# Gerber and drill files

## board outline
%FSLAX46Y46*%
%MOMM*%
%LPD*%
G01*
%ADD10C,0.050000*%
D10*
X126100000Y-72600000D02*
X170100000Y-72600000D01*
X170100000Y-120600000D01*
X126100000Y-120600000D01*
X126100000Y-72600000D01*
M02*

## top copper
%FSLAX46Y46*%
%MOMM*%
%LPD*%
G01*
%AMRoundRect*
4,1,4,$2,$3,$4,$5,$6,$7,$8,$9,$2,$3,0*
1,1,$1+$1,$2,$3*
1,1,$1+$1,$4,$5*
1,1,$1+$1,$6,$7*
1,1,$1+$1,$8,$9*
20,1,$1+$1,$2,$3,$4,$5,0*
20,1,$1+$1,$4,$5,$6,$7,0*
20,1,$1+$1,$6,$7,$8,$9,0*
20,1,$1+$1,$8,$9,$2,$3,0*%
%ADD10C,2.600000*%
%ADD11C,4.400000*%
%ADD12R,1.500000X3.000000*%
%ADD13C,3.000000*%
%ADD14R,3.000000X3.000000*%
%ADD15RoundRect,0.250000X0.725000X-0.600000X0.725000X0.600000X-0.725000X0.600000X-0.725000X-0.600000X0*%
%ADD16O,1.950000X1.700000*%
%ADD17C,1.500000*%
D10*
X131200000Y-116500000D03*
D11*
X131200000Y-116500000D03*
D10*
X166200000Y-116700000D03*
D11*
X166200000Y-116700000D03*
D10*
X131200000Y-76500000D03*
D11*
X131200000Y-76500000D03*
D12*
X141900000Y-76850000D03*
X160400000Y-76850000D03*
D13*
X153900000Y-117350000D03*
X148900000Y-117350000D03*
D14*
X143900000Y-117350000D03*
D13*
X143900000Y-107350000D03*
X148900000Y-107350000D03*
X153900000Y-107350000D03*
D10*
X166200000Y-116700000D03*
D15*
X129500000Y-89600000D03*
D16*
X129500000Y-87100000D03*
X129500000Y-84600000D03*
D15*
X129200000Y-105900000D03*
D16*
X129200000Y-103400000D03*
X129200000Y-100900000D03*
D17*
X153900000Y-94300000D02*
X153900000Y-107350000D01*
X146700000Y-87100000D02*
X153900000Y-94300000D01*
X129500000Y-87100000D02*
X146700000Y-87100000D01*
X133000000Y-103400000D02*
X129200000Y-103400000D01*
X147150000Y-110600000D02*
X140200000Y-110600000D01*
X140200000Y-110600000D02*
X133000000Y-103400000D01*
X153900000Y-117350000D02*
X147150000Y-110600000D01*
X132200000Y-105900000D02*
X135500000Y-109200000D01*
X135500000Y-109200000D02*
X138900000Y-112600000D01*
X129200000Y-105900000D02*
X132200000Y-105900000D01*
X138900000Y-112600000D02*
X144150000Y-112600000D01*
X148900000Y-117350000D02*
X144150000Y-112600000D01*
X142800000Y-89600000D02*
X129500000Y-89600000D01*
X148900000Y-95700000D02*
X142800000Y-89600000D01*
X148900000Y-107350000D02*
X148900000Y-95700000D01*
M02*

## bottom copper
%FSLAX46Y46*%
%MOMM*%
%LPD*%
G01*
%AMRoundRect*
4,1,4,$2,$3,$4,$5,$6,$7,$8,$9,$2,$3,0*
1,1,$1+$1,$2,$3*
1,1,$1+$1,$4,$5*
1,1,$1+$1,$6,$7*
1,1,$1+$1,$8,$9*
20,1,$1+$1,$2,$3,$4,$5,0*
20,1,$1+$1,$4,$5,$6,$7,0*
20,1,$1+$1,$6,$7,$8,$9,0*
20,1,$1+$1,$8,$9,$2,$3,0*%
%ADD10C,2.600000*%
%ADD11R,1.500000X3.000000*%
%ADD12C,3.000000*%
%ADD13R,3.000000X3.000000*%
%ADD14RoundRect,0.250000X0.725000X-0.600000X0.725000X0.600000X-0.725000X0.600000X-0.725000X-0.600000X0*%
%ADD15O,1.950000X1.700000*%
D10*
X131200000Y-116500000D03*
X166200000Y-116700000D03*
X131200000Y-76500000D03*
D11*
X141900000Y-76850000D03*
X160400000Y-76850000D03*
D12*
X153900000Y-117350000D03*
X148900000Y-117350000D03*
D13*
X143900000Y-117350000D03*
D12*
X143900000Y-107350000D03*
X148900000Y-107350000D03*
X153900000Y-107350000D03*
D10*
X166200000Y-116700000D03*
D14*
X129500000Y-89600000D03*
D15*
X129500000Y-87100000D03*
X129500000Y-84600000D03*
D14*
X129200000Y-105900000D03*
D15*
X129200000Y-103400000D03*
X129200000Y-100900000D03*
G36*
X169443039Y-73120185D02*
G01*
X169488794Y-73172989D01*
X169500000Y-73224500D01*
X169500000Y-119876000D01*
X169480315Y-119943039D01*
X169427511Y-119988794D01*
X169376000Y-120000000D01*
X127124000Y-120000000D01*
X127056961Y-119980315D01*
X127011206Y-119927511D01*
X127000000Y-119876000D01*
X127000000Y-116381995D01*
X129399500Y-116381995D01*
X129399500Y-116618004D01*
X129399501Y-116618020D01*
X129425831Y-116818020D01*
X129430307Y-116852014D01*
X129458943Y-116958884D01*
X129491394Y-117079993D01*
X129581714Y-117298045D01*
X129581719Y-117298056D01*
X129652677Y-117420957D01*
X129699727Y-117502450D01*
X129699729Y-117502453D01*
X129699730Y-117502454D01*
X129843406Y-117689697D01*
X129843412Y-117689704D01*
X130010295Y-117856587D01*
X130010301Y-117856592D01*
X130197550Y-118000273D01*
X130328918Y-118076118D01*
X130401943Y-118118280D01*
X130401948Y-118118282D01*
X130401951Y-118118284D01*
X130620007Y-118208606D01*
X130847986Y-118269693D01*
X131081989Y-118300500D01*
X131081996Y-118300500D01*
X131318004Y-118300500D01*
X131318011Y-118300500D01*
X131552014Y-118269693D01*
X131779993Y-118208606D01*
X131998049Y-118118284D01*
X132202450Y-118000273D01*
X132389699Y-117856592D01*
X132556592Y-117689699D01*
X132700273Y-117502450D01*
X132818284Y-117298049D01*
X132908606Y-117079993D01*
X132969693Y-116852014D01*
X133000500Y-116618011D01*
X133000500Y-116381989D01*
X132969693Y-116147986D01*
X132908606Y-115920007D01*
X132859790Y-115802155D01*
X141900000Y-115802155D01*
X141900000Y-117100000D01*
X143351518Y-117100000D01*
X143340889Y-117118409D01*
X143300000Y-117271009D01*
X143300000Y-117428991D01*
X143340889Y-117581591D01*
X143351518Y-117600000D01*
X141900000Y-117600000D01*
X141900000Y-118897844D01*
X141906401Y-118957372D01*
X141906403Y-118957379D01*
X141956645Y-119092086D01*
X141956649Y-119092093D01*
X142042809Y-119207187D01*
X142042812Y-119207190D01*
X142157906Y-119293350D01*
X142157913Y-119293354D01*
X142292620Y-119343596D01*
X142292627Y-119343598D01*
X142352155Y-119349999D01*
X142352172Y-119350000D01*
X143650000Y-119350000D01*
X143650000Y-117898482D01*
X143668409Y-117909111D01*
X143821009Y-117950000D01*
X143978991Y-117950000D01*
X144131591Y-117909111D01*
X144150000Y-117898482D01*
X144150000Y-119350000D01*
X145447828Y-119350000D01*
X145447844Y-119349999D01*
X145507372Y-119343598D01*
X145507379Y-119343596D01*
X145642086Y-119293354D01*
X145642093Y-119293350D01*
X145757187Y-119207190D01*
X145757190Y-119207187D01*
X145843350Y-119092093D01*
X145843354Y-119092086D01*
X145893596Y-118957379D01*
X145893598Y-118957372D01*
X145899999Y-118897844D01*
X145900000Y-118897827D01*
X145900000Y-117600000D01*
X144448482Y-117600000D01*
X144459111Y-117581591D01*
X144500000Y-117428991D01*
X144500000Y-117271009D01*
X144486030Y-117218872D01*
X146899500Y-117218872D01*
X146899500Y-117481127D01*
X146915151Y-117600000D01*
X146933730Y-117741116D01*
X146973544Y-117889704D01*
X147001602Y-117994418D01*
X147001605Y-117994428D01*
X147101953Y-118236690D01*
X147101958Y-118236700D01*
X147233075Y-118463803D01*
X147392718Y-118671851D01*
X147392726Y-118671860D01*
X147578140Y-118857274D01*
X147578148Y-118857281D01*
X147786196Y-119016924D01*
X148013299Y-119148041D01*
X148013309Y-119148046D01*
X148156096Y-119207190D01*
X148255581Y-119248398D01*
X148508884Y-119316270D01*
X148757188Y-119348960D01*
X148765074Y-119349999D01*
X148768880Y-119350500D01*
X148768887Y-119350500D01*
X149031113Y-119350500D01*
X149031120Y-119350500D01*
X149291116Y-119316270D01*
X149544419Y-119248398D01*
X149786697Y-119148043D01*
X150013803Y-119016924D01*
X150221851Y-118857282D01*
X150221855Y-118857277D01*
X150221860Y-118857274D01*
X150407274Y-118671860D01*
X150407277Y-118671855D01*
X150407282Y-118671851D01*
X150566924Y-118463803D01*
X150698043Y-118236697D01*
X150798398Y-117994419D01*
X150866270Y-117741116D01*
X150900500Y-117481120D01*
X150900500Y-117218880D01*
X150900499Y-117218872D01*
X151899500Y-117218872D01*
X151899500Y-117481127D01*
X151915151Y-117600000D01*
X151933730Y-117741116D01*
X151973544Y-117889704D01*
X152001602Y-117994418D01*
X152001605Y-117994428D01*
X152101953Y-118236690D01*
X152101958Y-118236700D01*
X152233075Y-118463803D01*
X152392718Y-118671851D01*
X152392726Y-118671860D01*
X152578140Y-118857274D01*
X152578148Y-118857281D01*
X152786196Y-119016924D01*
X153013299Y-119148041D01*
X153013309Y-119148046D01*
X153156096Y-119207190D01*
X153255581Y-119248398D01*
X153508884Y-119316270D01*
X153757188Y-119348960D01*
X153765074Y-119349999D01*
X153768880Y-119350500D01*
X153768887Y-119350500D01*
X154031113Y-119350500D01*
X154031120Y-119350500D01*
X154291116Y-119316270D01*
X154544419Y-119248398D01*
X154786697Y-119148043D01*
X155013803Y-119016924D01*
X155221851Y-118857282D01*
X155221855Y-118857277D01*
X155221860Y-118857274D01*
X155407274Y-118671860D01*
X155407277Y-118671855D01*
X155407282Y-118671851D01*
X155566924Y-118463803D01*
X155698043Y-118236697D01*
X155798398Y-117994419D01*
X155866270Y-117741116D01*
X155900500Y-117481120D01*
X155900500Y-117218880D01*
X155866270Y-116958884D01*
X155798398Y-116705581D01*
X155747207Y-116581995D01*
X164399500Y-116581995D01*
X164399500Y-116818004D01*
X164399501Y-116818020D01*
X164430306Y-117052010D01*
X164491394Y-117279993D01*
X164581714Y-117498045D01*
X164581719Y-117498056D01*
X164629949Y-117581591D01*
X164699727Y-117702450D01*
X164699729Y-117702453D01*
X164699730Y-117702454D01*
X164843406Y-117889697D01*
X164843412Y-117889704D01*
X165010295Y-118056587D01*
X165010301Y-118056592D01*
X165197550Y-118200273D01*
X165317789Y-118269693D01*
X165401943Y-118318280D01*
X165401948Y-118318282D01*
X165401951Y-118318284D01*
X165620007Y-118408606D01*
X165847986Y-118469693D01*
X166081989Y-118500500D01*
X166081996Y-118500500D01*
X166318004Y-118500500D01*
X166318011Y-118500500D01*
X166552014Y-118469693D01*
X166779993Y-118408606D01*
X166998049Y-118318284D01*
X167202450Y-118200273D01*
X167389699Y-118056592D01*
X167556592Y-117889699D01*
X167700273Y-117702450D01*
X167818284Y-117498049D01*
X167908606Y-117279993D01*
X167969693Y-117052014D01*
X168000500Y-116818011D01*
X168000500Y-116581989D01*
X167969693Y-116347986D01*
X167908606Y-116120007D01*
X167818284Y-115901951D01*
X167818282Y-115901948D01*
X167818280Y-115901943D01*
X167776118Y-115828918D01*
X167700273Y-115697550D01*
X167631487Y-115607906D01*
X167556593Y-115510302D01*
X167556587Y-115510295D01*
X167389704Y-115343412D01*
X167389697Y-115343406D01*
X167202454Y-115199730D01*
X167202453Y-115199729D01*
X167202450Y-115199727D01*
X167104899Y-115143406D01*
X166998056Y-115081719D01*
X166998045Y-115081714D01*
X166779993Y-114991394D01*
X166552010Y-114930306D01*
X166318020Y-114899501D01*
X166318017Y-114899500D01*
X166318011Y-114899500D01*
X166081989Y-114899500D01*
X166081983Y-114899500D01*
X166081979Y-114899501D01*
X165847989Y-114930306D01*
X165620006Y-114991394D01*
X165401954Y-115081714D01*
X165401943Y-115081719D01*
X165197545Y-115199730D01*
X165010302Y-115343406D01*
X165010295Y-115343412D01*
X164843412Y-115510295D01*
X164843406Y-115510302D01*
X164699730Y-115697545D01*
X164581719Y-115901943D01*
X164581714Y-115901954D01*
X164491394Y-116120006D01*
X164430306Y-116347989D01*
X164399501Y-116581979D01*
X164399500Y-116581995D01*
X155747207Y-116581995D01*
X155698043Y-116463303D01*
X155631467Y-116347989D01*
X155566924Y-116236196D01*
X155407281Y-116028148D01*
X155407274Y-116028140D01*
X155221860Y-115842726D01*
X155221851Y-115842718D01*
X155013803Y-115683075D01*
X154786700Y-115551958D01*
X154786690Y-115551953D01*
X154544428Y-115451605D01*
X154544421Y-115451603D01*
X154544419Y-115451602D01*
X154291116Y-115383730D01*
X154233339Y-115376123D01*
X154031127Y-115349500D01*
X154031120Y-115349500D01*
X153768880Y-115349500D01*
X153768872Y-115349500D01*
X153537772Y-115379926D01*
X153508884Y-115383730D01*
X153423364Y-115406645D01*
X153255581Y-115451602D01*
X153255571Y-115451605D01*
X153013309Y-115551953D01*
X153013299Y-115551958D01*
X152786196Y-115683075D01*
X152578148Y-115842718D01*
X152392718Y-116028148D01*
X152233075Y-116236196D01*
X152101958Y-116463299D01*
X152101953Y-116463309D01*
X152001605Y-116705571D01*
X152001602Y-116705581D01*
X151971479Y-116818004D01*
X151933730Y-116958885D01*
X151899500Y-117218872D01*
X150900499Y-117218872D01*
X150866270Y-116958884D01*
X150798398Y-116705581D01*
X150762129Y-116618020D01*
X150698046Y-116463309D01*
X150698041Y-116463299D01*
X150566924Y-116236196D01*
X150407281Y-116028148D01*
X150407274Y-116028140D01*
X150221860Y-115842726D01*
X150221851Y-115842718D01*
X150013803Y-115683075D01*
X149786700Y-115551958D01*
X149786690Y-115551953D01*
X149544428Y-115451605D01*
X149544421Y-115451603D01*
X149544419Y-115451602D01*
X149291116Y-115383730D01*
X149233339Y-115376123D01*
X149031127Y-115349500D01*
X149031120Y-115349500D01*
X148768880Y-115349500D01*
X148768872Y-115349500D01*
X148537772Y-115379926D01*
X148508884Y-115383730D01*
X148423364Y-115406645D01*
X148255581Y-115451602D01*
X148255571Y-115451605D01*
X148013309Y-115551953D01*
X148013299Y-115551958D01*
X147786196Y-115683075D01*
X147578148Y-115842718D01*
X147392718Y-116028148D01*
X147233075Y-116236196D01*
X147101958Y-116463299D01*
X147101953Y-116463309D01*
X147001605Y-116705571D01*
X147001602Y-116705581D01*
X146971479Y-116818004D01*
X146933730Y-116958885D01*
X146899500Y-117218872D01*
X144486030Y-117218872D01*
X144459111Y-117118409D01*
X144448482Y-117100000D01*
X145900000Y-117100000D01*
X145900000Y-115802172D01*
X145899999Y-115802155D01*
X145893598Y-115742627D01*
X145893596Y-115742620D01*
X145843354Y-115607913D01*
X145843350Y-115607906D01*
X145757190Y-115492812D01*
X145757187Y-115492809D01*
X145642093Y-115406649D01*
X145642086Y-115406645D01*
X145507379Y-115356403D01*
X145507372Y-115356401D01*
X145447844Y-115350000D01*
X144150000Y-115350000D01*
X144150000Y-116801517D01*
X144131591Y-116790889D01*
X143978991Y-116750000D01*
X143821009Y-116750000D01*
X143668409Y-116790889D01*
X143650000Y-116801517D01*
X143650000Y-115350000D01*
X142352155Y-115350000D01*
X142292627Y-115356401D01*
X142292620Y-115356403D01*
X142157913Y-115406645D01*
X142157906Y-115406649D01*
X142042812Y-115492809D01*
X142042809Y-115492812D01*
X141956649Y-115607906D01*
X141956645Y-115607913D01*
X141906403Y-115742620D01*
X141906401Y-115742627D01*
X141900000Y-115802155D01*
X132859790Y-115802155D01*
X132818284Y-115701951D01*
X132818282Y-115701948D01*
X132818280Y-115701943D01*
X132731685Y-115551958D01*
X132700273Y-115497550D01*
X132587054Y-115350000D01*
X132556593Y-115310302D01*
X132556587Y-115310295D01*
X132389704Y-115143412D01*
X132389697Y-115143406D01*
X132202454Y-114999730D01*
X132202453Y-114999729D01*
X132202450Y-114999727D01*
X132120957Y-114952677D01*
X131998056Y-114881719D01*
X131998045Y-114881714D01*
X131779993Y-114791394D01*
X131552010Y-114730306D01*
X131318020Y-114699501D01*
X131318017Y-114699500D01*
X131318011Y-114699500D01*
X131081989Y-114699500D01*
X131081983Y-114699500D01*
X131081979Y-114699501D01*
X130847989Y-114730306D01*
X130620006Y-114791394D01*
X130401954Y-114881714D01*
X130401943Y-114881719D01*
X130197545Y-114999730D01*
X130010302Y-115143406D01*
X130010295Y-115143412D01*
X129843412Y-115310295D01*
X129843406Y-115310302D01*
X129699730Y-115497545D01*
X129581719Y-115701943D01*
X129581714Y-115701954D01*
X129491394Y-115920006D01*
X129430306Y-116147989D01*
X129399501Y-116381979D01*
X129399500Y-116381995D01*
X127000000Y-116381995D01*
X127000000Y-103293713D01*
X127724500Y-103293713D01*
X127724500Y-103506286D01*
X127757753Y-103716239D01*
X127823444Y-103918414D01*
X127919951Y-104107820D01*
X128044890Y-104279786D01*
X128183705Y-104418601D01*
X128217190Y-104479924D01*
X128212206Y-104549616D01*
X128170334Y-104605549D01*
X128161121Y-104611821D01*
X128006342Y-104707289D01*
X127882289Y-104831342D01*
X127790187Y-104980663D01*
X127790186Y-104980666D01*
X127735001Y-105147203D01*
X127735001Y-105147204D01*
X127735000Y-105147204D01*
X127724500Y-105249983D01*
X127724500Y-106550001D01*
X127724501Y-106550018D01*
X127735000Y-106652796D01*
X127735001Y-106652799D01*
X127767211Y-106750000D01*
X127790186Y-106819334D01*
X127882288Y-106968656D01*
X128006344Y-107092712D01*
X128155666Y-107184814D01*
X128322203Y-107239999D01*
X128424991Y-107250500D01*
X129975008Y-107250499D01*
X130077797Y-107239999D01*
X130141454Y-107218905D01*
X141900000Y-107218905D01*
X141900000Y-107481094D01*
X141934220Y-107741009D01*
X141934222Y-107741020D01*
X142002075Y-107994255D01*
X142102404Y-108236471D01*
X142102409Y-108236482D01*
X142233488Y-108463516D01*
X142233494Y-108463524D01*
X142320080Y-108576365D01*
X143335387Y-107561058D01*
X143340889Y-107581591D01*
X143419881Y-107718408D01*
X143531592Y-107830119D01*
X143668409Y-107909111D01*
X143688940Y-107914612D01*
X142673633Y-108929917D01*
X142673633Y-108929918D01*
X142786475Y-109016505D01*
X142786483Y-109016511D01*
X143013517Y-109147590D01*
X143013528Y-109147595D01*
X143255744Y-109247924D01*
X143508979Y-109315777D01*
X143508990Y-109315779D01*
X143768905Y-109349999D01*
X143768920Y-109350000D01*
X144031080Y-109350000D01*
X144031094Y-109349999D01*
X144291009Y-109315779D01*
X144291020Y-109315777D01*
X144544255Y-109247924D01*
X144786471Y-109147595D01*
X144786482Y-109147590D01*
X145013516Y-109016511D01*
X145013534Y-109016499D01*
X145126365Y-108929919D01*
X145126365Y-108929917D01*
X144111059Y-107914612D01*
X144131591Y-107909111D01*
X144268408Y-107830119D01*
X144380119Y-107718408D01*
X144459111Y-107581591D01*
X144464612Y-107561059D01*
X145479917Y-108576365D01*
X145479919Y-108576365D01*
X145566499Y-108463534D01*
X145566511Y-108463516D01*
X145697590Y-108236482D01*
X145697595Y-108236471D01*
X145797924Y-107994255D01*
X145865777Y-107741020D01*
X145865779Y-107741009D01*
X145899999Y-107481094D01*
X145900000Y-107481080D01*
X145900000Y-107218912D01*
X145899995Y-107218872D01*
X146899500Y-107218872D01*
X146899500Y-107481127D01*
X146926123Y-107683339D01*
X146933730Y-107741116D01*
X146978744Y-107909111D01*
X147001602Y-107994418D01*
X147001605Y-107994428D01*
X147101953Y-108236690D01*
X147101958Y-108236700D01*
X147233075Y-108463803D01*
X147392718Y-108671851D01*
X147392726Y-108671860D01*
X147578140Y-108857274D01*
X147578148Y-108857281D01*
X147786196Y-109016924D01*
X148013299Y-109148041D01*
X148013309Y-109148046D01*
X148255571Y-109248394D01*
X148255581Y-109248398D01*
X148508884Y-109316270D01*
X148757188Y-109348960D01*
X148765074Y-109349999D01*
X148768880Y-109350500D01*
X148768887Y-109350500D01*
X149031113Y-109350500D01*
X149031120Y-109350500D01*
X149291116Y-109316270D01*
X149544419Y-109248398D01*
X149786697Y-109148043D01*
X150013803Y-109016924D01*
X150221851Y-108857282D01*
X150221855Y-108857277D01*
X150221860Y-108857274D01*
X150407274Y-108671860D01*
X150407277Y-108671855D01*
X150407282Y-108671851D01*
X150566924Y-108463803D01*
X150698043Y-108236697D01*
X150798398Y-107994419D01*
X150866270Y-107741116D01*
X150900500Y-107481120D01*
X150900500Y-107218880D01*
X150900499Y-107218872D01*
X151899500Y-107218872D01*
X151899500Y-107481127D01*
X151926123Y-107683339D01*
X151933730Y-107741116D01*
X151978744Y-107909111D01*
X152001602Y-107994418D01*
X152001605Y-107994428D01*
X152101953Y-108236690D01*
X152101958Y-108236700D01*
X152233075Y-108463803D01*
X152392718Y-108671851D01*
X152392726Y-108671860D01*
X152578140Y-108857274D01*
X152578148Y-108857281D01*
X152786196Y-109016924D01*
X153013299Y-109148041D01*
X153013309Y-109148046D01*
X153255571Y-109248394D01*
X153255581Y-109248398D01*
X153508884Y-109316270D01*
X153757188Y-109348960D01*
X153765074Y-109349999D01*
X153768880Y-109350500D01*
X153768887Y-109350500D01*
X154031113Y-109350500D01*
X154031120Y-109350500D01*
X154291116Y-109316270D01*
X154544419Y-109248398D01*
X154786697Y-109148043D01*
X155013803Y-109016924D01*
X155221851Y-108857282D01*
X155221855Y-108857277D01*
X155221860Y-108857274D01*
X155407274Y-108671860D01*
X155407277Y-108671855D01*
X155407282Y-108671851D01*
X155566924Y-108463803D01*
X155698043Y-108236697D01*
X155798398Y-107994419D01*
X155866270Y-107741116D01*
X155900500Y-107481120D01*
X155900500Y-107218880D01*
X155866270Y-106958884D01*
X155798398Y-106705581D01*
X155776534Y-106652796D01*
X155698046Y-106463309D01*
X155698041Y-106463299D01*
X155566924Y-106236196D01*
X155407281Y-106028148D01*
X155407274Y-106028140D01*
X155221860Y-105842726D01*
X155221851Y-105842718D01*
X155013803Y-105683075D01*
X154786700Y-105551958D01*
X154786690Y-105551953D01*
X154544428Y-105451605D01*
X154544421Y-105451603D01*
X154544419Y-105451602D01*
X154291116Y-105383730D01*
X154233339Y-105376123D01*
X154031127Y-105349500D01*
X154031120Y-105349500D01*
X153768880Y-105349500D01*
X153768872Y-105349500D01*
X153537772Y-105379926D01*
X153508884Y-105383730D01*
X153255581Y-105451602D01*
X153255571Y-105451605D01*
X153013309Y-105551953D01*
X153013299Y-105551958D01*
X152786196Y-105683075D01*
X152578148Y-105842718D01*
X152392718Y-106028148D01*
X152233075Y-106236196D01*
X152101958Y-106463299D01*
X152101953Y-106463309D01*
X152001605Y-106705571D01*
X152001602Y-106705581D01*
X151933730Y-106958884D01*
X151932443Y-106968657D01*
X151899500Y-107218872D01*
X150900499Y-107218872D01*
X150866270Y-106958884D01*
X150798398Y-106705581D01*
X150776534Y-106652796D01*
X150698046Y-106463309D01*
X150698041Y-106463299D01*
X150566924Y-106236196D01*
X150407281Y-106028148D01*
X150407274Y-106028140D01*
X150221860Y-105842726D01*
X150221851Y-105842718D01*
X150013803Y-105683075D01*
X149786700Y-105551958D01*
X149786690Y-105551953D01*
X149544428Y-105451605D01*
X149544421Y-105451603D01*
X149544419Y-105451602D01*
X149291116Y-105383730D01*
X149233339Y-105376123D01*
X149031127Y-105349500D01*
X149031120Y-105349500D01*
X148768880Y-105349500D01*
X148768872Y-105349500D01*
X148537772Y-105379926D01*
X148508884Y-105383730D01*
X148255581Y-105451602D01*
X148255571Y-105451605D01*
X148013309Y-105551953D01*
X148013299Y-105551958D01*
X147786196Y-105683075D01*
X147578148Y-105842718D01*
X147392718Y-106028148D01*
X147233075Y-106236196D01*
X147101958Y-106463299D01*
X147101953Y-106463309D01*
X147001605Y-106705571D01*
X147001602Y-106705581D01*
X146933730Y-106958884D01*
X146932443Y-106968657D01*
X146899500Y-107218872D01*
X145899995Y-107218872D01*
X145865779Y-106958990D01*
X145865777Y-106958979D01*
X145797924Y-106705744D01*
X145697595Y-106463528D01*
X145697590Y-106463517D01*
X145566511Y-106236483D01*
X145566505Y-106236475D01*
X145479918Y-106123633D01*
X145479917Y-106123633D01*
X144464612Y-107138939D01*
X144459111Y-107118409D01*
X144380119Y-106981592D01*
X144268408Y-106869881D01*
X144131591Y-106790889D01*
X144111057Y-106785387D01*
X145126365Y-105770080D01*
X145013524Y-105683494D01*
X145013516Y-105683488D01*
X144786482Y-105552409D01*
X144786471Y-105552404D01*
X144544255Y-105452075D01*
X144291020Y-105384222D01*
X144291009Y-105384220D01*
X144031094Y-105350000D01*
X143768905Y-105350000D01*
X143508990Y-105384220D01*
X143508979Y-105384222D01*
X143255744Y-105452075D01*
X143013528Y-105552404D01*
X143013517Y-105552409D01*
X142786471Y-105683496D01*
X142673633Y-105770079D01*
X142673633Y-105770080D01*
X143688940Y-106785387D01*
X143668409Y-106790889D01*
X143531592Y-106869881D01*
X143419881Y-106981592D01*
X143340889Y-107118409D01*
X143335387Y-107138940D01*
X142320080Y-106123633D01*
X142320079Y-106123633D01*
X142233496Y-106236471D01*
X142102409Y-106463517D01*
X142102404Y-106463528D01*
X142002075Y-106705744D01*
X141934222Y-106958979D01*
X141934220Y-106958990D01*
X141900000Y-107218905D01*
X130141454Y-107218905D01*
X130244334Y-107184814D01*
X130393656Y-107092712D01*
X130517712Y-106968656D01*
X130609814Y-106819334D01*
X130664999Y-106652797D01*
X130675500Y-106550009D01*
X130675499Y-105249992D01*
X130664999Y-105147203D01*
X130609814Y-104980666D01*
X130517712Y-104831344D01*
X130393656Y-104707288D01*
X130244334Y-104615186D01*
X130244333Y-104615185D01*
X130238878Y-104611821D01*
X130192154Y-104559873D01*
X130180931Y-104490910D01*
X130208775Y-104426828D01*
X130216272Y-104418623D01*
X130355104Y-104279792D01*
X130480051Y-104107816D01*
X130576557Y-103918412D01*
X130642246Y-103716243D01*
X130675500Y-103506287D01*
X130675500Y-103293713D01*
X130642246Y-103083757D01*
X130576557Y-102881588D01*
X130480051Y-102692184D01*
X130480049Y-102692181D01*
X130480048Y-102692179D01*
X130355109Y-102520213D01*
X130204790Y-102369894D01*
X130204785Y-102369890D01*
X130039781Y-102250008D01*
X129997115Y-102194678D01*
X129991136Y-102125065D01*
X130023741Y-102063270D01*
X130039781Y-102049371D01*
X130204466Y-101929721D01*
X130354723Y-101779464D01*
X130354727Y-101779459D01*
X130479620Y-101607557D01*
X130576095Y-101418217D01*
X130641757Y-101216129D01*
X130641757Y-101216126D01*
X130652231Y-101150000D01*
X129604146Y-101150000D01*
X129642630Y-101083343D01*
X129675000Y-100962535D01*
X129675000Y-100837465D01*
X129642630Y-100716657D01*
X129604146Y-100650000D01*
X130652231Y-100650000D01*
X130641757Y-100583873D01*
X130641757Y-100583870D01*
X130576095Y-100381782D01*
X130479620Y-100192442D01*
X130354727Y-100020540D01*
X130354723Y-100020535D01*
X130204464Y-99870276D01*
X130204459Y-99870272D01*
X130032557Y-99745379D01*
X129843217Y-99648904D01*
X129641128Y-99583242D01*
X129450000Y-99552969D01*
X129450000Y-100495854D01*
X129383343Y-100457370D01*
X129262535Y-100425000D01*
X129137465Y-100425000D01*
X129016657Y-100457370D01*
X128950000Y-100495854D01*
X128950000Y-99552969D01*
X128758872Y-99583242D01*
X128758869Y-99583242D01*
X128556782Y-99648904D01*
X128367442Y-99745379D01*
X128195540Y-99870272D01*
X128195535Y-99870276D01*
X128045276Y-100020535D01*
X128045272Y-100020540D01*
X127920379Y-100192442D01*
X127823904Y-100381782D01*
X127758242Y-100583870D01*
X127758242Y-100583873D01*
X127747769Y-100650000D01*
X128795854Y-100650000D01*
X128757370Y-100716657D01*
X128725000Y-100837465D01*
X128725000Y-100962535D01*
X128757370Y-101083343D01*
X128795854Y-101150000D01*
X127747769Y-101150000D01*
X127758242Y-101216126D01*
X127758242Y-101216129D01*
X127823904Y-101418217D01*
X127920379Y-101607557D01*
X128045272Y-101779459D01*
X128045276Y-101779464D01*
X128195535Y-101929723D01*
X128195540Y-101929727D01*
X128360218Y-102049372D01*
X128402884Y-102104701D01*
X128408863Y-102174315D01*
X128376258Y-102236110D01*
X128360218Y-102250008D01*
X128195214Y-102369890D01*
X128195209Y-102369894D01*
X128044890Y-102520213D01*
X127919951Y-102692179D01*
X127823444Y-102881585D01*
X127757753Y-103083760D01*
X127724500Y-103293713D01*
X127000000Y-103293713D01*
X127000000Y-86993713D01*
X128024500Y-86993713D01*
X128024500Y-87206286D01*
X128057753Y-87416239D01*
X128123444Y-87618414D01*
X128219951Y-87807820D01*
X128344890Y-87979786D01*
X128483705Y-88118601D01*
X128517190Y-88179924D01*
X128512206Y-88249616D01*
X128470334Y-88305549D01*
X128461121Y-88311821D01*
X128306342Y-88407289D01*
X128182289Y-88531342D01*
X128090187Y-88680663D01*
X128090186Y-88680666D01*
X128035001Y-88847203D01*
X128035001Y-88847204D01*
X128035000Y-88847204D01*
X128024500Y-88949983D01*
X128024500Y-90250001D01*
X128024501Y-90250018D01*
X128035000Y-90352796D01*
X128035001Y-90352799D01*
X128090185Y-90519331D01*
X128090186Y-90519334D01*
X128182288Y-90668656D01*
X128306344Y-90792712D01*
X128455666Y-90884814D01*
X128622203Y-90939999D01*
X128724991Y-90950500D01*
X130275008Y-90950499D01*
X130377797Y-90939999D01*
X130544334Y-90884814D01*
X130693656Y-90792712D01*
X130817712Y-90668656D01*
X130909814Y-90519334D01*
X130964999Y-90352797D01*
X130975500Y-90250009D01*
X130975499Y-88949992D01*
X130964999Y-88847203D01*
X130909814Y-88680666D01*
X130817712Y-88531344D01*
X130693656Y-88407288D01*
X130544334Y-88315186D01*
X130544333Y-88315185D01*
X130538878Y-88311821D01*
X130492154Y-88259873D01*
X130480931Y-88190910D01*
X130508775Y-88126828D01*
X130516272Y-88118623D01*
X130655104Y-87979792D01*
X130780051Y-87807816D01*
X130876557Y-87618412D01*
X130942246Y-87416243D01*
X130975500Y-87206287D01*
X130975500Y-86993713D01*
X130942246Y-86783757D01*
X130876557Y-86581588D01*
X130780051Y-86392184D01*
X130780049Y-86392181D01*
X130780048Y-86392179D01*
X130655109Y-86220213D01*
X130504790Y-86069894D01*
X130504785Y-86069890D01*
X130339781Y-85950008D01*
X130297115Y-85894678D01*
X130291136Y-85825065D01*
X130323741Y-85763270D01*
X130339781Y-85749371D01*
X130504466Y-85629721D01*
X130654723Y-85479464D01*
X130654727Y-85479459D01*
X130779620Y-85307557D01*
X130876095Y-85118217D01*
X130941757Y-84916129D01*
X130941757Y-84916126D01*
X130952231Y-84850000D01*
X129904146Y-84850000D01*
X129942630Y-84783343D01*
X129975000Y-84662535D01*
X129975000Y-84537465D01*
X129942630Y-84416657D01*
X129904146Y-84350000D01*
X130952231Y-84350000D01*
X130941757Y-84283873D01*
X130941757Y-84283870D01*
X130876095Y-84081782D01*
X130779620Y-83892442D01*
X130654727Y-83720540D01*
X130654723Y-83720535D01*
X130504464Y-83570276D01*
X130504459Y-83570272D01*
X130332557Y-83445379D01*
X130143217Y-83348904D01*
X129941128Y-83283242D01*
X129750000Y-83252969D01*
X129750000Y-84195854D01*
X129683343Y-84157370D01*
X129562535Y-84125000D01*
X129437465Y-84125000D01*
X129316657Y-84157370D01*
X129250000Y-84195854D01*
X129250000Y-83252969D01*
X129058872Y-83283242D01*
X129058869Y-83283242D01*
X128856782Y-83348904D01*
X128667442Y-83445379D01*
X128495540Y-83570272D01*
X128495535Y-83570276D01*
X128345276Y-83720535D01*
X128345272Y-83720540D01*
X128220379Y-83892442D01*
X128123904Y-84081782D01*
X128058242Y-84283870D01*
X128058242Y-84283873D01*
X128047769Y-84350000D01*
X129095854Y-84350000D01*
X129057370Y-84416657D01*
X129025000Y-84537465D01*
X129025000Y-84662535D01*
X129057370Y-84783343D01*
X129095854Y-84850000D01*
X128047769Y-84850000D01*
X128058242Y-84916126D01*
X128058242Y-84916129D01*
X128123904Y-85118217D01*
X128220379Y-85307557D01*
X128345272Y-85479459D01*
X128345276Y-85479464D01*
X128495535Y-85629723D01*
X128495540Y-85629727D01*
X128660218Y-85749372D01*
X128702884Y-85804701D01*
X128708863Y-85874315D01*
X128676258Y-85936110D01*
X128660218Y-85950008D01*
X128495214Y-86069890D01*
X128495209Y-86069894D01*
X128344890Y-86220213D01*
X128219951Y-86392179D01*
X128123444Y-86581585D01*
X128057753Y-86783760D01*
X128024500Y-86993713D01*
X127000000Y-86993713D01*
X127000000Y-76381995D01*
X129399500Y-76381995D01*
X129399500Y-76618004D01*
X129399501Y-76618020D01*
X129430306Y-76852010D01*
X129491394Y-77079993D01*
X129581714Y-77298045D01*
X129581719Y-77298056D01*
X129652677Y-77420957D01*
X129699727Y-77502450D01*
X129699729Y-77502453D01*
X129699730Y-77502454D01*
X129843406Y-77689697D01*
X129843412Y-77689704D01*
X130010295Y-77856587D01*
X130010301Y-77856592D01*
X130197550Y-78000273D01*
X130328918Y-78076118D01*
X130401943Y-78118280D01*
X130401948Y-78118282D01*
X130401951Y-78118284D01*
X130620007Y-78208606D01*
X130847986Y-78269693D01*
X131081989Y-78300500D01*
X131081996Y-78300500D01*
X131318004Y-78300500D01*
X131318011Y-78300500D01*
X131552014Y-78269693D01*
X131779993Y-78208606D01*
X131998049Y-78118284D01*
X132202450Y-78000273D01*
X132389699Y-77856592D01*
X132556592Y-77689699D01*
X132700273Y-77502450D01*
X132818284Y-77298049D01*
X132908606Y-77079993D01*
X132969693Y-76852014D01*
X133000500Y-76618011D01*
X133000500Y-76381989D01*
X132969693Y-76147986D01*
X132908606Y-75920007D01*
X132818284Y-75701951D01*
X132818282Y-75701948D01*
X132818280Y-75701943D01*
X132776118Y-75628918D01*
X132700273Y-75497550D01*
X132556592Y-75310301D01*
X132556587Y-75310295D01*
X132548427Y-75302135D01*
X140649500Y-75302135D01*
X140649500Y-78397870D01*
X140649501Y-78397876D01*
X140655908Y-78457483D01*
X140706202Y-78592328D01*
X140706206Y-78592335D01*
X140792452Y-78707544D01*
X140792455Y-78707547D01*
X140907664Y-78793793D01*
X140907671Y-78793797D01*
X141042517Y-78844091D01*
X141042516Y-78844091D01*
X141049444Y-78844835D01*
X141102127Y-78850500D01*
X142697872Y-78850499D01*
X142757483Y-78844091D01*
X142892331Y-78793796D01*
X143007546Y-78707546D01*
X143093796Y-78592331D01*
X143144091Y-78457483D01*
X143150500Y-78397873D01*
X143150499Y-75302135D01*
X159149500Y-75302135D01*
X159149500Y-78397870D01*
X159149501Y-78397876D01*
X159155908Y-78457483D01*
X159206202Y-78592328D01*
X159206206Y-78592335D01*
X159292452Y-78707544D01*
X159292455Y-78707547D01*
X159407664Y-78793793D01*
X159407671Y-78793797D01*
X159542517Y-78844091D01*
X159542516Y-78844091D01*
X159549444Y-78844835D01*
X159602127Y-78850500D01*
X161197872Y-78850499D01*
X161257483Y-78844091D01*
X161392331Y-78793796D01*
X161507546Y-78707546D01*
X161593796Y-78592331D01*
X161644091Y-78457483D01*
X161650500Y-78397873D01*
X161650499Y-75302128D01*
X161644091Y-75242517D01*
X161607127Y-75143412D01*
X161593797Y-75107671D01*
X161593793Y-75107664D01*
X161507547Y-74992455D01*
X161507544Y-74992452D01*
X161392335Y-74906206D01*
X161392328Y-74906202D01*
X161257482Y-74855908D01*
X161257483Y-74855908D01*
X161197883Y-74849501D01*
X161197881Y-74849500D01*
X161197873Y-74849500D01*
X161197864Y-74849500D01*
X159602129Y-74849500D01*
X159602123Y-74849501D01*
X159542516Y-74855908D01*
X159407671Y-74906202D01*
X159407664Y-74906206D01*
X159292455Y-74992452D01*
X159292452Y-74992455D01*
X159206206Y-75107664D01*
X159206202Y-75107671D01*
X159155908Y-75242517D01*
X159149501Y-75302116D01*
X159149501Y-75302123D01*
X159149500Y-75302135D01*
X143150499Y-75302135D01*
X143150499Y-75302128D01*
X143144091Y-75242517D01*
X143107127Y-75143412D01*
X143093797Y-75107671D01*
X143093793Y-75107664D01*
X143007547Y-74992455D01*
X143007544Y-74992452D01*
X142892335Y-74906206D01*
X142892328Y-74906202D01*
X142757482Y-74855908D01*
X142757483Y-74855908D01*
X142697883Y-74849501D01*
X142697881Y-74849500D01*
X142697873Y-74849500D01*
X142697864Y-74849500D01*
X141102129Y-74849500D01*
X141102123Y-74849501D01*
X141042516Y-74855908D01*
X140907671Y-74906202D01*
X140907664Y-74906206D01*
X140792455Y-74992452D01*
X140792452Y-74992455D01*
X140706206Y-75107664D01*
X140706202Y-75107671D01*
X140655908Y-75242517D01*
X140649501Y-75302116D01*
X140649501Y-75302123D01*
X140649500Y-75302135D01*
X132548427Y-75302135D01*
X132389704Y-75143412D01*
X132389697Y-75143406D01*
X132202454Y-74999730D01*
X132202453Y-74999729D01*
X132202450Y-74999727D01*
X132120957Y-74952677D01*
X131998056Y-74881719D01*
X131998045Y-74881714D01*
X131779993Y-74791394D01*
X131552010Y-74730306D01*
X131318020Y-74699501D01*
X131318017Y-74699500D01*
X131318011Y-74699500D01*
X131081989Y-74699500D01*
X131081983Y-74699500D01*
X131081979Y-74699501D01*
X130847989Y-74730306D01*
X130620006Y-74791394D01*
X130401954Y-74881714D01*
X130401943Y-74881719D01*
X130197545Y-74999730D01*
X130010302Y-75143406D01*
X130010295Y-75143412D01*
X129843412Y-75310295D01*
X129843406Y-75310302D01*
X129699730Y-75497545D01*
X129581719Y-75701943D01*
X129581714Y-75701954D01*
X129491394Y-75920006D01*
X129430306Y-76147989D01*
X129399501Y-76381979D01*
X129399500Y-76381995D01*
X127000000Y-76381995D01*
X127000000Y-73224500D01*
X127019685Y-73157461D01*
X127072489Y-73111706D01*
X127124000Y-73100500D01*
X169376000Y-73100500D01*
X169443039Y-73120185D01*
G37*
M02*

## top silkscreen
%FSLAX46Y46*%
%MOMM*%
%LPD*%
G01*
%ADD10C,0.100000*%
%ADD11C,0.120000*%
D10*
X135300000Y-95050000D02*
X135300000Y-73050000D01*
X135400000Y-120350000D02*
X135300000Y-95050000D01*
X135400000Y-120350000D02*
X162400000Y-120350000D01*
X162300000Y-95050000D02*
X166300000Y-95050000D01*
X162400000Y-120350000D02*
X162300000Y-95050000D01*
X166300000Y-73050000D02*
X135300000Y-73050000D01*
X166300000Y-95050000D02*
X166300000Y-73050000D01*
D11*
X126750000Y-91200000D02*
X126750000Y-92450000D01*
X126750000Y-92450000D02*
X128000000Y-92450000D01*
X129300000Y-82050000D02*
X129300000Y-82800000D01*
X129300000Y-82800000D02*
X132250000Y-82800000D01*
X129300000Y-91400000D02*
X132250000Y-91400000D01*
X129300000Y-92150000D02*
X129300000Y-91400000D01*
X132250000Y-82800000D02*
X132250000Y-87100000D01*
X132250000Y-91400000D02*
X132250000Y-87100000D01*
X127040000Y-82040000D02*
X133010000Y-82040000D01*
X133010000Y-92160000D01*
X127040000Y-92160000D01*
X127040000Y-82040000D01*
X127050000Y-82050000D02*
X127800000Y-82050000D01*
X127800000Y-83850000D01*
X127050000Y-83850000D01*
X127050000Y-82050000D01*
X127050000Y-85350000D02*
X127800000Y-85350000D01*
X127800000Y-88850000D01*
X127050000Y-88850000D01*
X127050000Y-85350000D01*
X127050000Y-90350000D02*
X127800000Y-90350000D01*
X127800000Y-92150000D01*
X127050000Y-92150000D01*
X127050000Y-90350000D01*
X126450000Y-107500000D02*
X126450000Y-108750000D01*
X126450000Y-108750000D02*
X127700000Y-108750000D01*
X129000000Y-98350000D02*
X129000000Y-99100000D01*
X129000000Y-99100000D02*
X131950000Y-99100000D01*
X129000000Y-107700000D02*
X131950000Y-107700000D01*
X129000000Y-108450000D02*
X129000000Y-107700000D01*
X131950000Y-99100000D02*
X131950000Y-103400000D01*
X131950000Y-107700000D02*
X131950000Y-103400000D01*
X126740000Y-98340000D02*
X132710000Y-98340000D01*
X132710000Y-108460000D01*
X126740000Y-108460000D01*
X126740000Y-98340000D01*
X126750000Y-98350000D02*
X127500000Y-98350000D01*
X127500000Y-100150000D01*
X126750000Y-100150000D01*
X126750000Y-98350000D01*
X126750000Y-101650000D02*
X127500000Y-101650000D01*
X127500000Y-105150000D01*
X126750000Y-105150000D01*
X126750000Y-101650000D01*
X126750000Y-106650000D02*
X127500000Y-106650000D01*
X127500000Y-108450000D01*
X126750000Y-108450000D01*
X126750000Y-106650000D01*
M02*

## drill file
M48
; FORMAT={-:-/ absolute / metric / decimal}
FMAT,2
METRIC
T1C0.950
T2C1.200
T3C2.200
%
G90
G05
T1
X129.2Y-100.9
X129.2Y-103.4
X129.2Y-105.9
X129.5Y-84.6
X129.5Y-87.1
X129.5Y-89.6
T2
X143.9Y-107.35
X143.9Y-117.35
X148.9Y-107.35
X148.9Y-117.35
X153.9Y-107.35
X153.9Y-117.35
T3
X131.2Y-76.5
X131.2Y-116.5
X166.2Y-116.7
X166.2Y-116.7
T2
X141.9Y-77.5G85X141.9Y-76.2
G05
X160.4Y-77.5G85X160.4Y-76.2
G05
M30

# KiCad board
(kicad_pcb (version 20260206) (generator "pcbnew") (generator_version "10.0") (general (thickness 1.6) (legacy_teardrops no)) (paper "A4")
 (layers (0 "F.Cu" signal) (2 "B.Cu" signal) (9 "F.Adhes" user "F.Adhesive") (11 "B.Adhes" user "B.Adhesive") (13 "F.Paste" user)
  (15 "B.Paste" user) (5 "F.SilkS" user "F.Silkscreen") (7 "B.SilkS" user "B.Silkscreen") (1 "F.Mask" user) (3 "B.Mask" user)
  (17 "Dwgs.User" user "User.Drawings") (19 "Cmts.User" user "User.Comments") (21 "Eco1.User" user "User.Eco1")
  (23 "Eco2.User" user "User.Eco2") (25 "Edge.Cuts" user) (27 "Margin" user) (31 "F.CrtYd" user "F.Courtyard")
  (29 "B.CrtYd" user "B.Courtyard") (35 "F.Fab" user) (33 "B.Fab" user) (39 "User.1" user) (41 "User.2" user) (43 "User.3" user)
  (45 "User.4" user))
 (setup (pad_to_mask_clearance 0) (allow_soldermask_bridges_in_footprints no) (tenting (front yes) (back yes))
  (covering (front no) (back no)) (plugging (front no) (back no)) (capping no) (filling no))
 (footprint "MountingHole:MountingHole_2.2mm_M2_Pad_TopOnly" (layer "F.Cu") (at 131.2 116.5)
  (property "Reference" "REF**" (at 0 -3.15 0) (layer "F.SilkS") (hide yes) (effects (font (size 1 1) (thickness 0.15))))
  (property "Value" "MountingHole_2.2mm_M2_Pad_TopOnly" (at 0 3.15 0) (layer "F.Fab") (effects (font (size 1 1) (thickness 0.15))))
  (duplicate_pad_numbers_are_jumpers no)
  (pad "1" thru_hole circle (at 0 0) (size 2.6 2.6) (drill 2.2) (layers "*.Cu" "*.Mask") (remove_unused_layers no) (zone_connect 2))
  (pad "1" connect circle (at 0 0) (size 4.4 4.4) (layers "F.Cu" "F.Mask") (zone_connect 2)))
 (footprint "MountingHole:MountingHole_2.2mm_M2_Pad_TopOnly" (layer "F.Cu") (at 166.2 116.7)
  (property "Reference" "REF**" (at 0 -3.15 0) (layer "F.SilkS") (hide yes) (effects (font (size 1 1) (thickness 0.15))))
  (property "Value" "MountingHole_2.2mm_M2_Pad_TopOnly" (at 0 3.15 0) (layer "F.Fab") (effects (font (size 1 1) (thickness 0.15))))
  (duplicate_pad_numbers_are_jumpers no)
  (pad "1" thru_hole circle (at 0 0) (size 2.6 2.6) (drill 2.2) (layers "*.Cu" "*.Mask") (remove_unused_layers no) (zone_connect 2))
  (pad "1" connect circle (at 0 0) (size 4.4 4.4) (layers "F.Cu" "F.Mask") (zone_connect 2)))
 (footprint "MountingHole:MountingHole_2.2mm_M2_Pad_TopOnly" (layer "F.Cu") (at 131.2 76.5)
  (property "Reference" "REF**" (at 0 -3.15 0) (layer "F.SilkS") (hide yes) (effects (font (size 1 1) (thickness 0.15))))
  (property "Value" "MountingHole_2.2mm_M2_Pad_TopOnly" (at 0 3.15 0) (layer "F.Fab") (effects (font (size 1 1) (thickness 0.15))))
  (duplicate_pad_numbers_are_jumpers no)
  (pad "1" thru_hole circle (at 0 0) (size 2.6 2.6) (drill 2.2) (layers "*.Cu" "*.Mask") (remove_unused_layers no) (zone_connect 2))
  (pad "1" connect circle (at 0 0) (size 4.4 4.4) (layers "F.Cu" "F.Mask") (zone_connect 2)))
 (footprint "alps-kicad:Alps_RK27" (layer "F.Cu") (at 143.9 118.35 90)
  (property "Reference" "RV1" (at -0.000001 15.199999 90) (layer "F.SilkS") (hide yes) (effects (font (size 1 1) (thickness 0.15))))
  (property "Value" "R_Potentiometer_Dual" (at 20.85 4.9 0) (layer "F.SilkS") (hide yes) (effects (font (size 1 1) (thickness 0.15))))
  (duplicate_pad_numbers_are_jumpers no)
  (fp_line (start 23.3 -8.6) (end 45.3 -8.6) (stroke (width 0.1) (type default)) (layer "F.SilkS"))
  (fp_line (start -2 -8.5) (end 23.3 -8.6) (stroke (width 0.1) (type default)) (layer "F.SilkS"))
  (fp_line (start -2 -8.5) (end -2 18.5) (stroke (width 0.1) (type default)) (layer "F.SilkS"))
  (fp_line (start 23.3 18.4) (end 23.3 22.4) (stroke (width 0.1) (type default)) (layer "F.SilkS"))
  (fp_line (start -2 18.5) (end 23.3 18.4) (stroke (width 0.1) (type default)) (layer "F.SilkS"))
  (fp_line (start 45.3 22.4) (end 45.3 -8.6) (stroke (width 0.1) (type default)) (layer "F.SilkS"))
  (fp_line (start 23.3 22.4) (end 45.3 22.4) (stroke (width 0.1) (type default)) (layer "F.SilkS"))
  (pad "" thru_hole rect (at 41.5 -2 90) (size 3 1.5) (drill oval 2.5 1.2) (layers "*.Cu" "*.Mask") (remove_unused_layers no)
   (thermal_bridge_angle 45))
  (pad "" thru_hole rect (at 41.5 16.5 90) (size 3 1.5) (drill oval 2.5 1.2) (layers "*.Cu" "*.Mask") (remove_unused_layers no)
   (thermal_bridge_angle 45))
  (pad "1" thru_hole circle (at 1 10 270) (size 3 3) (drill 1.2) (layers "*.Cu" "*.Mask") (remove_unused_layers no) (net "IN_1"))
  (pad "2" thru_hole circle (at 1 5 270) (size 3 3) (drill 1.2) (layers "*.Cu" "*.Mask") (remove_unused_layers no) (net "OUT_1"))
  (pad "3" thru_hole rect (at 1 0 270) (size 3 3) (drill 1.2) (layers "*.Cu" "*.Mask") (remove_unused_layers no) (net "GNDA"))
  (pad "4" thru_hole circle (at 11 0 270) (size 3 3) (drill 1.2) (layers "*.Cu" "*.Mask") (remove_unused_layers no) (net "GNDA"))
  (pad "5" thru_hole circle (at 11 5 270) (size 3 3) (drill 1.2) (layers "*.Cu" "*.Mask") (remove_unused_layers no) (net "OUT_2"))
  (pad "6" thru_hole circle (at 11 10 270) (size 3 3) (drill 1.2) (layers "*.Cu" "*.Mask") (remove_unused_layers no) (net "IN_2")))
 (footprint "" (layer "F.Cu") (at 166.2 116.7)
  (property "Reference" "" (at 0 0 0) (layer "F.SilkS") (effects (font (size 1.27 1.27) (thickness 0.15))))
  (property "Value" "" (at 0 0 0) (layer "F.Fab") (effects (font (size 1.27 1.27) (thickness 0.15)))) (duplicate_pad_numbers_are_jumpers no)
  (pad "1" thru_hole circle (at 0 0) (size 2.6 2.6) (drill 2.2) (layers "*.Cu" "*.Mask") (remove_unused_layers no) (zone_connect 2)))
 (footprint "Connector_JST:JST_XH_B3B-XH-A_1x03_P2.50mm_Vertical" (layer "F.Cu") (at 129.5 89.6 90)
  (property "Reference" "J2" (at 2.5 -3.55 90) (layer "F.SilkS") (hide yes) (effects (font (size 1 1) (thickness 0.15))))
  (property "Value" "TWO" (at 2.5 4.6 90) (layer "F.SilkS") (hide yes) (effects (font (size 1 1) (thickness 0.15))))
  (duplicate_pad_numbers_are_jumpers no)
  (fp_line (start -1.6 -2.75) (end -2.85 -2.75) (stroke (width 0.12) (type solid)) (layer "F.SilkS"))
  (fp_line (start -2.85 -2.75) (end -2.85 -1.5) (stroke (width 0.12) (type solid)) (layer "F.SilkS"))
  (fp_line (start 7.55 -0.2) (end 6.8 -0.2) (stroke (width 0.12) (type solid)) (layer "F.SilkS"))
  (fp_line (start 6.8 -0.2) (end 6.8 2.75) (stroke (width 0.12) (type solid)) (layer "F.SilkS"))
  (fp_line (start -1.8 -0.2) (end -1.8 2.75) (stroke (width 0.12) (type solid)) (layer "F.SilkS"))
  (fp_line (start -2.55 -0.2) (end -1.8 -0.2) (stroke (width 0.12) (type solid)) (layer "F.SilkS"))
  (fp_line (start 6.8 2.75) (end 2.5 2.75) (stroke (width 0.12) (type solid)) (layer "F.SilkS"))
  (fp_line (start -1.8 2.75) (end 2.5 2.75) (stroke (width 0.12) (type solid)) (layer "F.SilkS"))
  (fp_rect (start -2.56 -2.46) (end 7.56 3.51) (stroke (width 0.12) (type solid)) (fill no) (layer "F.SilkS"))
  (fp_rect (start 5.75 -2.45) (end 7.55 -1.7) (stroke (width 0.12) (type solid)) (fill no) (layer "F.SilkS"))
  (fp_rect (start 0.75 -2.45) (end 4.25 -1.7) (stroke (width 0.12) (type solid)) (fill no) (layer "F.SilkS"))
  (fp_rect (start -2.55 -2.45) (end -0.75 -1.7) (stroke (width 0.12) (type solid)) (fill no) (layer "F.SilkS"))
  (pad "1" thru_hole roundrect (at 0 0 90) (size 1.7 1.95) (drill 0.95) (layers "*.Cu" "*.Mask") (remove_unused_layers no)
   (roundrect_rratio 0.147059) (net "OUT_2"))
  (pad "2" thru_hole oval (at 2.5 0 90) (size 1.7 1.95) (drill 0.95) (layers "*.Cu" "*.Mask") (remove_unused_layers no) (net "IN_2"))
  (pad "3" thru_hole oval (at 5 0 90) (size 1.7 1.95) (drill 0.95) (layers "*.Cu" "*.Mask") (remove_unused_layers no) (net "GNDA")))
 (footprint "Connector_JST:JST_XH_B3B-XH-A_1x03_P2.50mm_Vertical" (layer "F.Cu") (at 129.2 105.9 90)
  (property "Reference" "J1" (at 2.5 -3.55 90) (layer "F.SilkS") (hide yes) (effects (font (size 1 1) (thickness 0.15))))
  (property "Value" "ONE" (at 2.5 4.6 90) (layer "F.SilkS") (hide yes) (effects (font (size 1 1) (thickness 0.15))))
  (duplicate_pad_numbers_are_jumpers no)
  (fp_line (start -1.6 -2.75) (end -2.85 -2.75) (stroke (width 0.12) (type solid)) (layer "F.SilkS"))
  (fp_line (start -2.85 -2.75) (end -2.85 -1.5) (stroke (width 0.12) (type solid)) (layer "F.SilkS"))
  (fp_line (start 7.55 -0.2) (end 6.8 -0.2) (stroke (width 0.12) (type solid)) (layer "F.SilkS"))
  (fp_line (start 6.8 -0.2) (end 6.8 2.75) (stroke (width 0.12) (type solid)) (layer "F.SilkS"))
  (fp_line (start -1.8 -0.2) (end -1.8 2.75) (stroke (width 0.12) (type solid)) (layer "F.SilkS"))
  (fp_line (start -2.55 -0.2) (end -1.8 -0.2) (stroke (width 0.12) (type solid)) (layer "F.SilkS"))
  (fp_line (start 6.8 2.75) (end 2.5 2.75) (stroke (width 0.12) (type solid)) (layer "F.SilkS"))
  (fp_line (start -1.8 2.75) (end 2.5 2.75) (stroke (width 0.12) (type solid)) (layer "F.SilkS"))
  (fp_rect (start -2.56 -2.46) (end 7.56 3.51) (stroke (width 0.12) (type solid)) (fill no) (layer "F.SilkS"))
  (fp_rect (start 5.75 -2.45) (end 7.55 -1.7) (stroke (width 0.12) (type solid)) (fill no) (layer "F.SilkS"))
  (fp_rect (start 0.75 -2.45) (end 4.25 -1.7) (stroke (width 0.12) (type solid)) (fill no) (layer "F.SilkS"))
  (fp_rect (start -2.55 -2.45) (end -0.75 -1.7) (stroke (width 0.12) (type solid)) (fill no) (layer "F.SilkS"))
  (pad "1" thru_hole roundrect (at 0 0 90) (size 1.7 1.95) (drill 0.95) (layers "*.Cu" "*.Mask") (remove_unused_layers no)
   (roundrect_rratio 0.147059) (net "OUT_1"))
  (pad "2" thru_hole oval (at 2.5 0 90) (size 1.7 1.95) (drill 0.95) (layers "*.Cu" "*.Mask") (remove_unused_layers no) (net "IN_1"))
  (pad "3" thru_hole oval (at 5 0 90) (size 1.7 1.95) (drill 0.95) (layers "*.Cu" "*.Mask") (remove_unused_layers no) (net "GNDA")))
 (gr_rect (start 126.1 72.6) (end 170.1 120.6) (stroke (width 0.05) (type default)) (fill no) (layer "Edge.Cuts"))
 (segment (start 153.9 94.3) (end 153.9 107.35) (width 1.5) (layer "F.Cu") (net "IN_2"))
 (segment (start 146.7 87.1) (end 153.9 94.3) (width 1.5) (layer "F.Cu") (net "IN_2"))
 (segment (start 129.5 87.1) (end 146.7 87.1) (width 1.5) (layer "F.Cu") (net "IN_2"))
 (segment (start 133 103.4) (end 129.2 103.4) (width 1.5) (layer "F.Cu") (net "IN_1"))
 (segment (start 147.15 110.6) (end 140.2 110.6) (width 1.5) (layer "F.Cu") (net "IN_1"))
 (segment (start 140.2 110.6) (end 133 103.4) (width 1.5) (layer "F.Cu") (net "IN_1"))
 (segment (start 153.9 117.35) (end 147.15 110.6) (width 1.5) (layer "F.Cu") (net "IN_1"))
 (segment (start 132.2 105.9) (end 135.5 109.2) (width 1.5) (layer "F.Cu") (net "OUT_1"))
 (segment (start 135.5 109.2) (end 138.9 112.6) (width 1.5) (layer "F.Cu") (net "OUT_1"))
 (segment (start 129.2 105.9) (end 132.2 105.9) (width 1.5) (layer "F.Cu") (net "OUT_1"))
 (segment (start 138.9 112.6) (end 144.15 112.6) (width 1.5) (layer "F.Cu") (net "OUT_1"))
 (segment (start 148.9 117.35) (end 144.15 112.6) (width 1.5) (layer "F.Cu") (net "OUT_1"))
 (segment (start 142.8 89.6) (end 129.5 89.6) (width 1.5) (layer "F.Cu") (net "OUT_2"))
 (segment (start 148.9 95.7) (end 142.8 89.6) (width 1.5) (layer "F.Cu") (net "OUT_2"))
 (segment (start 148.9 107.35) (end 148.9 95.7) (width 1.5) (layer "F.Cu") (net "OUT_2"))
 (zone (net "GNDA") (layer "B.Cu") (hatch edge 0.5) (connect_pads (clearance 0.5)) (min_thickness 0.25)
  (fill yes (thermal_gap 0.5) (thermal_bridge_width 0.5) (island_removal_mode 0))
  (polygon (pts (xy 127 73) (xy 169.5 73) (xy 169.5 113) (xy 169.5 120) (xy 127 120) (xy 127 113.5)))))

